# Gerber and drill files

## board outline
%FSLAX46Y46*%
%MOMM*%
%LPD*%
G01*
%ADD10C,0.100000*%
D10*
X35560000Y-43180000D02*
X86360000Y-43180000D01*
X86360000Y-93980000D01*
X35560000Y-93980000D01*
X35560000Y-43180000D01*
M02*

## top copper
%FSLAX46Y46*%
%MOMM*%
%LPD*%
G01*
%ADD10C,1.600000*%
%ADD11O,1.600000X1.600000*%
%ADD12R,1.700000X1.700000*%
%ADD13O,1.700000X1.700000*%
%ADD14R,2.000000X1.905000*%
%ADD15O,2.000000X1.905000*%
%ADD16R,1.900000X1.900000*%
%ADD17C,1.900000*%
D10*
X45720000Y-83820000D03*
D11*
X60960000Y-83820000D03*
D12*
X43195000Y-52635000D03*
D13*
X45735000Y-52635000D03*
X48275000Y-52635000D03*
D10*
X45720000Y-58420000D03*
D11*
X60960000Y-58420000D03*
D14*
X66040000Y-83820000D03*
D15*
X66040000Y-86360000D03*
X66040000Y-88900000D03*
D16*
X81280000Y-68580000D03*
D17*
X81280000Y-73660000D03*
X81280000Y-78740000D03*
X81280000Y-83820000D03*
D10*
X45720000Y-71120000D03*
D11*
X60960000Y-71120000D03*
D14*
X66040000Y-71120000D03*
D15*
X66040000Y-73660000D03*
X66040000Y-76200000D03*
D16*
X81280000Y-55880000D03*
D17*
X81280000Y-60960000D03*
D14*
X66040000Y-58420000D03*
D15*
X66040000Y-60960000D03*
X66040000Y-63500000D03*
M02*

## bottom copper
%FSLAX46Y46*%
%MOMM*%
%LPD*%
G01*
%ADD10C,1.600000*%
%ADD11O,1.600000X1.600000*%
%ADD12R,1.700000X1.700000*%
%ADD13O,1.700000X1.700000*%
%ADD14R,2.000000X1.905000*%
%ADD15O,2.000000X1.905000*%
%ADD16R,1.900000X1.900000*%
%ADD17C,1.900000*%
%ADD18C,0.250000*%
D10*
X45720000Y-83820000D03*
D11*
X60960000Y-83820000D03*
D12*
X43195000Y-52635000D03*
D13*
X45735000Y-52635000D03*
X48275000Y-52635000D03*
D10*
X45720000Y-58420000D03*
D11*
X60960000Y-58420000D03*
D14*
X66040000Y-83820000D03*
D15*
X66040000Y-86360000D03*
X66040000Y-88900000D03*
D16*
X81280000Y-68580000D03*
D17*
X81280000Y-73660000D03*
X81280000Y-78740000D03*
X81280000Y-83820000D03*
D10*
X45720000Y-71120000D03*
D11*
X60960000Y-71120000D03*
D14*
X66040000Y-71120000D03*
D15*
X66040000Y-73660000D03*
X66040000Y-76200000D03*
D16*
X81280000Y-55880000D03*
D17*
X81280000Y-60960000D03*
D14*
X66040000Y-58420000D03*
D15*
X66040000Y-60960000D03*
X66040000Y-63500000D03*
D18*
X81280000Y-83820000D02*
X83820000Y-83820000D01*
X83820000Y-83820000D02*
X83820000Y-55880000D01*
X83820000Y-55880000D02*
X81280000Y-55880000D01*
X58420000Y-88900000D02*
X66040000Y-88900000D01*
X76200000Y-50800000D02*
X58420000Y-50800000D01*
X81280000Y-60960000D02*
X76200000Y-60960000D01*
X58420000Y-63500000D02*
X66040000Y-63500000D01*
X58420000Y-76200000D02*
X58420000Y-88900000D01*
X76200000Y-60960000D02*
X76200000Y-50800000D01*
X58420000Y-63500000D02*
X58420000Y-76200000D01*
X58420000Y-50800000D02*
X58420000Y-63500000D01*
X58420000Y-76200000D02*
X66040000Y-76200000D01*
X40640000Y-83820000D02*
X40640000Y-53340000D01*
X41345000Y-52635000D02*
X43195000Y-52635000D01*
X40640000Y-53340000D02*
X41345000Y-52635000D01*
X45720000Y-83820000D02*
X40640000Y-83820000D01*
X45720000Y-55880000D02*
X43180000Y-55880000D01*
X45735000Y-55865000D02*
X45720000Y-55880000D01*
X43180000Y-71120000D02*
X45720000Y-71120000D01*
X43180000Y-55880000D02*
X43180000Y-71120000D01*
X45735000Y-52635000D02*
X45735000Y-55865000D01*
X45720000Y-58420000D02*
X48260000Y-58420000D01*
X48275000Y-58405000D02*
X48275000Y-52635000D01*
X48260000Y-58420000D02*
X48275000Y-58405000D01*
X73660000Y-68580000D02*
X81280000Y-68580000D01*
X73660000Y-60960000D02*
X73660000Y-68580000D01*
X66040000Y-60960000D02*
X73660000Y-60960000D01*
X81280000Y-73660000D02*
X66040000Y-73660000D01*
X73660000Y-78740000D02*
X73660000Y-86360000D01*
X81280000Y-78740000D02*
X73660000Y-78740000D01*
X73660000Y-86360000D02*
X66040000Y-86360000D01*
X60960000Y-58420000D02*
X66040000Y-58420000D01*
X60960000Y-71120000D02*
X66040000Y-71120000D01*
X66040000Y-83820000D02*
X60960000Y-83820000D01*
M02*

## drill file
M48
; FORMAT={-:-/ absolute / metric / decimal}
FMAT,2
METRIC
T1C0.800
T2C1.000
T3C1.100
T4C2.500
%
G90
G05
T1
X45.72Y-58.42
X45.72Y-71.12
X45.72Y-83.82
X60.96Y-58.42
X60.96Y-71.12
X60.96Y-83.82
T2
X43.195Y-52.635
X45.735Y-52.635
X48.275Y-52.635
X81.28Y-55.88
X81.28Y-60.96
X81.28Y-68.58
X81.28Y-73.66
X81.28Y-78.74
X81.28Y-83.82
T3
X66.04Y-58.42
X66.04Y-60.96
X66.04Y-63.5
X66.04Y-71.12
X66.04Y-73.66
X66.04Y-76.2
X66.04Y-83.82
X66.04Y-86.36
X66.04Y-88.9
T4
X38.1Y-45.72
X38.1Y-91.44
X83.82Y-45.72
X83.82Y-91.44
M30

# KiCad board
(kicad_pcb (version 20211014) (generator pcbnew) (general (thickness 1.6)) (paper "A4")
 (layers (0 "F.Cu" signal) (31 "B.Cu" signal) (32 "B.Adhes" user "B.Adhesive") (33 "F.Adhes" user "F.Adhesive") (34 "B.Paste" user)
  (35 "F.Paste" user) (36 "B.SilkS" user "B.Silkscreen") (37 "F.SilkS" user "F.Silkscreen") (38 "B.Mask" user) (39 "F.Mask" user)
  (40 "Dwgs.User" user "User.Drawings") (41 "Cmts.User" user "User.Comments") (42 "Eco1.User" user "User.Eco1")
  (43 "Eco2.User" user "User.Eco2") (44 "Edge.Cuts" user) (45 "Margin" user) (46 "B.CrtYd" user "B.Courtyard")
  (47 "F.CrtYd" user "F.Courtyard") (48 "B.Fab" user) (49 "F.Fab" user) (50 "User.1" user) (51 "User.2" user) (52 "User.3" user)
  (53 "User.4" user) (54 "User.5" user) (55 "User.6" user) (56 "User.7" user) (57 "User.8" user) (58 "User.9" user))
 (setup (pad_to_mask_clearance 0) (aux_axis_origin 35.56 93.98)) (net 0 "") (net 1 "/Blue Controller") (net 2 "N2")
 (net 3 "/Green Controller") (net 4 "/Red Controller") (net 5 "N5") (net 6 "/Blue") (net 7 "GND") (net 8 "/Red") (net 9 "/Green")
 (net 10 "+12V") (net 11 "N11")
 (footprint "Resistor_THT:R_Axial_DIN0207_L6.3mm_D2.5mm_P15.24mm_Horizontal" (layer "F.Cu") (at 45.72 83.82)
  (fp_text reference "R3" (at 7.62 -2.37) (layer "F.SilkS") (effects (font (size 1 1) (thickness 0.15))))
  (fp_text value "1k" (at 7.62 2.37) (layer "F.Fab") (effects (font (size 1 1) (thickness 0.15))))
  (pad "1" thru_hole circle (at 0 0) (size 1.6 1.6) (drill 0.8) (layers *.Cu *.Mask) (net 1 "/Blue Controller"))
  (pad "2" thru_hole oval (at 15.24 0) (size 1.6 1.6) (drill 0.8) (layers *.Cu *.Mask) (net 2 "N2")))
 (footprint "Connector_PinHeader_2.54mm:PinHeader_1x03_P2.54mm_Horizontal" (layer "F.Cu") (at 43.195 52.635 90)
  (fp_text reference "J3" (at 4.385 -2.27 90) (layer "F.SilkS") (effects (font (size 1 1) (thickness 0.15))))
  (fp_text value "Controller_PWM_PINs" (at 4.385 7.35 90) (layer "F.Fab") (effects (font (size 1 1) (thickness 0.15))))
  (pad "1" thru_hole rect (at 0 0 90) (size 1.7 1.7) (drill 1) (layers *.Cu *.Mask) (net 1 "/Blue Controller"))
  (pad "2" thru_hole oval (at 0 2.54 90) (size 1.7 1.7) (drill 1) (layers *.Cu *.Mask) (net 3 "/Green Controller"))
  (pad "3" thru_hole oval (at 0 5.08 90) (size 1.7 1.7) (drill 1) (layers *.Cu *.Mask) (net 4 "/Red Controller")))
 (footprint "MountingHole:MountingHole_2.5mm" (layer "F.Cu") (at 83.82 45.72)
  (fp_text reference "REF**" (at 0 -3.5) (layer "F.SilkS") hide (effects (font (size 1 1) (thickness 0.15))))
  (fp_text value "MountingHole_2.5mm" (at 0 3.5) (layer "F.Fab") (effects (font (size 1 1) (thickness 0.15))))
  (pad "" np_thru_hole circle (at 0 0) (size 2.5 2.5) (drill 2.5) (layers *.Cu *.Mask)))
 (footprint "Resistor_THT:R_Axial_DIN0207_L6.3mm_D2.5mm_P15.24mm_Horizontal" (layer "F.Cu") (at 45.72 58.42)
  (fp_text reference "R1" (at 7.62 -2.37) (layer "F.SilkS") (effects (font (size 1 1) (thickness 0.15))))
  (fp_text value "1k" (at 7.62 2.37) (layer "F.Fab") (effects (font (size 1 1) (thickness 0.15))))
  (pad "1" thru_hole circle (at 0 0) (size 1.6 1.6) (drill 0.8) (layers *.Cu *.Mask) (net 4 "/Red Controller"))
  (pad "2" thru_hole oval (at 15.24 0) (size 1.6 1.6) (drill 0.8) (layers *.Cu *.Mask) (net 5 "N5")))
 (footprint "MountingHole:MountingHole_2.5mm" (layer "F.Cu") (at 38.1 45.72)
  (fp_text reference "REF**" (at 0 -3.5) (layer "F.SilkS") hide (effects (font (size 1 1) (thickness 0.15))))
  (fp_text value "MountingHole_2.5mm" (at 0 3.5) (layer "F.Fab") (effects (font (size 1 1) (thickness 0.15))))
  (pad "" np_thru_hole circle (at 0 0) (size 2.5 2.5) (drill 2.5) (layers *.Mask)))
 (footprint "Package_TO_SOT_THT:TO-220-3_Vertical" (layer "F.Cu") (at 66.04 83.82 -90)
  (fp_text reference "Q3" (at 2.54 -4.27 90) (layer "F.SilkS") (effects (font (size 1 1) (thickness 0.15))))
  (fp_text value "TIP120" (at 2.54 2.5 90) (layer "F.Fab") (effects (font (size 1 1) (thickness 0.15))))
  (pad "1" thru_hole rect (at 0 0 270) (size 1.905 2) (drill 1.1) (layers *.Cu *.Mask) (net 2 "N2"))
  (pad "2" thru_hole oval (at 2.54 0 270) (size 1.905 2) (drill 1.1) (layers *.Cu *.Mask) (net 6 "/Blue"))
  (pad "3" thru_hole oval (at 5.08 0 270) (size 1.905 2) (drill 1.1) (layers *.Cu *.Mask) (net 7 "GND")))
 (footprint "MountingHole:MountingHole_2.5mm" (layer "F.Cu") (at 83.82 91.44)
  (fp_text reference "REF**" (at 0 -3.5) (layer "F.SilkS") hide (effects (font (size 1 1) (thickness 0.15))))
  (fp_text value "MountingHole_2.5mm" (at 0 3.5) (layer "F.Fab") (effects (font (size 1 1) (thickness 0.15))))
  (pad "" np_thru_hole circle (at 0 0) (size 2.5 2.5) (drill 2.5) (layers *.Cu *.Mask)))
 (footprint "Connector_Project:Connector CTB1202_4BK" (layer "F.Cu") (at 81.28 68.58 -90)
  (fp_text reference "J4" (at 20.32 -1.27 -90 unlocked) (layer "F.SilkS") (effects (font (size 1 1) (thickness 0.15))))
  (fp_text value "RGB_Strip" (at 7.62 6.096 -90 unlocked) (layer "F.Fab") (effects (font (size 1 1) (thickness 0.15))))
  (pad "1" thru_hole rect (at 0 0 270) (size 1.9 1.9) (drill 1) (layers *.Cu *.Mask) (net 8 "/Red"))
  (pad "2" thru_hole circle (at 5.08 0 270) (size 1.9 1.9) (drill 1) (layers *.Cu *.Mask) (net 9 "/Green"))
  (pad "3" thru_hole circle (at 10.16 0 270) (size 1.9 1.9) (drill 1) (layers *.Cu *.Mask) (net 6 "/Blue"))
  (pad "4" thru_hole circle (at 15.24 0 270) (size 1.9 1.9) (drill 1) (layers *.Cu *.Mask) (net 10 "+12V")))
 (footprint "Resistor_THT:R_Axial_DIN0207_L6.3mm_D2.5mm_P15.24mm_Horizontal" (layer "F.Cu") (at 45.72 71.12)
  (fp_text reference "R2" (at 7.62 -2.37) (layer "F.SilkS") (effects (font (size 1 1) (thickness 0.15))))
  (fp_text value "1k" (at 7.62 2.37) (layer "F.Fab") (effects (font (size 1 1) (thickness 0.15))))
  (pad "1" thru_hole circle (at 0 0) (size 1.6 1.6) (drill 0.8) (layers *.Cu *.Mask) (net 3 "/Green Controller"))
  (pad "2" thru_hole oval (at 15.24 0) (size 1.6 1.6) (drill 0.8) (layers *.Cu *.Mask) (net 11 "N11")))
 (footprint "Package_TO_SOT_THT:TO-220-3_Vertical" (layer "F.Cu") (at 66.04 71.12 -90)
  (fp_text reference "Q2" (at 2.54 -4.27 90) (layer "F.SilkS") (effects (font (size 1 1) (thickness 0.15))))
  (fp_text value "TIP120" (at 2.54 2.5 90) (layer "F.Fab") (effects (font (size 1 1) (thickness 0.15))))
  (pad "1" thru_hole rect (at 0 0 270) (size 1.905 2) (drill 1.1) (layers *.Cu *.Mask) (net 11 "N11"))
  (pad "2" thru_hole oval (at 2.54 0 270) (size 1.905 2) (drill 1.1) (layers *.Cu *.Mask) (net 9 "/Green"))
  (pad "3" thru_hole oval (at 5.08 0 270) (size 1.905 2) (drill 1.1) (layers *.Cu *.Mask) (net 7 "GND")))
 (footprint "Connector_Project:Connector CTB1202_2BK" (layer "F.Cu") (at 81.28 55.88 -90)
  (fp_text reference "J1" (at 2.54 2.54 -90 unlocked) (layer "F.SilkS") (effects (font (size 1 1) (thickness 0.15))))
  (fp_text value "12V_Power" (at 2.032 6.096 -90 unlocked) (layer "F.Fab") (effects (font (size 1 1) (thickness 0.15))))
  (pad "1" thru_hole rect (at 0 0 270) (size 1.9 1.9) (drill 1) (layers *.Cu *.Mask) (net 10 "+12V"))
  (pad "2" thru_hole circle (at 5.08 0 270) (size 1.9 1.9) (drill 1) (layers *.Cu *.Mask) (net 7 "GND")))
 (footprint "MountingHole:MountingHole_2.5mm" (layer "F.Cu") (at 38.1 91.44)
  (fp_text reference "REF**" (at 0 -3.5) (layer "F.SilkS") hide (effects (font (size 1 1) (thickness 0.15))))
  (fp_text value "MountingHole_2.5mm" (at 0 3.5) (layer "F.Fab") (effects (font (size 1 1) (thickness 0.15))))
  (pad "" np_thru_hole circle (at 0 0) (size 2.5 2.5) (drill 2.5) (layers *.Cu *.Mask)))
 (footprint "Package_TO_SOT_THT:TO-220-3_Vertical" (layer "F.Cu") (at 66.04 58.42 -90)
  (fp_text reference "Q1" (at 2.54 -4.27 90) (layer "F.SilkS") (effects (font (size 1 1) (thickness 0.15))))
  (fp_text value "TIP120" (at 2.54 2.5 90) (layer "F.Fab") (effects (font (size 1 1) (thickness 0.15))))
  (pad "1" thru_hole rect (at 0 0 270) (size 1.905 2) (drill 1.1) (layers *.Cu *.Mask) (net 5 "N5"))
  (pad "2" thru_hole oval (at 2.54 0 270) (size 1.905 2) (drill 1.1) (layers *.Cu *.Mask) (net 8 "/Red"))
  (pad "3" thru_hole oval (at 5.08 0 270) (size 1.905 2) (drill 1.1) (layers *.Cu *.Mask) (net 7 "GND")))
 (gr_rect (start 35.56 43.18) (end 86.36 93.98) (layer "Edge.Cuts") (width 0.1) (fill none))
 (segment (start 81.28 83.82) (end 83.82 83.82) (width 0.25) (layer "B.Cu") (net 10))
 (segment (start 83.82 83.82) (end 83.82 55.88) (width 0.25) (layer "B.Cu") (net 10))
 (segment (start 83.82 55.88) (end 81.28 55.88) (width 0.25) (layer "B.Cu") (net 10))
 (segment (start 58.42 88.9) (end 66.04 88.9) (width 0.25) (layer "B.Cu") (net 7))
 (segment (start 76.2 50.8) (end 58.42 50.8) (width 0.25) (layer "B.Cu") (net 7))
 (segment (start 81.28 60.96) (end 76.2 60.96) (width 0.25) (layer "B.Cu") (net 7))
 (segment (start 58.42 63.5) (end 66.04 63.5) (width 0.25) (layer "B.Cu") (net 7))
 (segment (start 58.42 76.2) (end 58.42 88.9) (width 0.25) (layer "B.Cu") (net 7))
 (segment (start 76.2 60.96) (end 76.2 50.8) (width 0.25) (layer "B.Cu") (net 7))
 (segment (start 58.42 63.5) (end 58.42 76.2) (width 0.25) (layer "B.Cu") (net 7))
 (segment (start 58.42 50.8) (end 58.42 63.5) (width 0.25) (layer "B.Cu") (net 7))
 (segment (start 58.42 76.2) (end 66.04 76.2) (width 0.25) (layer "B.Cu") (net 7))
 (segment (start 40.64 83.82) (end 40.64 53.34) (width 0.25) (layer "B.Cu") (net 1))
 (segment (start 41.345 52.635) (end 43.195 52.635) (width 0.25) (layer "B.Cu") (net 1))
 (segment (start 40.64 53.34) (end 41.345 52.635) (width 0.25) (layer "B.Cu") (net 1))
 (segment (start 45.72 83.82) (end 40.64 83.82) (width 0.25) (layer "B.Cu") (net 1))
 (segment (start 45.72 55.88) (end 43.18 55.88) (width 0.25) (layer "B.Cu") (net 3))
 (segment (start 45.735 55.865) (end 45.72 55.88) (width 0.25) (layer "B.Cu") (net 3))
 (segment (start 43.18 71.12) (end 45.72 71.12) (width 0.25) (layer "B.Cu") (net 3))
 (segment (start 43.18 55.88) (end 43.18 71.12) (width 0.25) (layer "B.Cu") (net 3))
 (segment (start 45.735 52.635) (end 45.735 55.865) (width 0.25) (layer "B.Cu") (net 3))
 (segment (start 45.72 58.42) (end 48.26 58.42) (width 0.25) (layer "B.Cu") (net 4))
 (segment (start 48.275 58.405) (end 48.275 52.635) (width 0.25) (layer "B.Cu") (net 4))
 (segment (start 48.26 58.42) (end 48.275 58.405) (width 0.25) (layer "B.Cu") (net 4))
 (segment (start 73.66 68.58) (end 81.28 68.58) (width 0.25) (layer "B.Cu") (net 8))
 (segment (start 73.66 60.96) (end 73.66 68.58) (width 0.25) (layer "B.Cu") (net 8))
 (segment (start 66.04 60.96) (end 73.66 60.96) (width 0.25) (layer "B.Cu") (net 8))
 (segment (start 81.28 73.66) (end 66.04 73.66) (width 0.25) (layer "B.Cu") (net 9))
 (segment (start 73.66 78.74) (end 73.66 86.36) (width 0.25) (layer "B.Cu") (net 6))
 (segment (start 81.28 78.74) (end 73.66 78.74) (width 0.25) (layer "B.Cu") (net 6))
 (segment (start 73.66 86.36) (end 66.04 86.36) (width 0.25) (layer "B.Cu") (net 6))
 (segment (start 60.96 58.42) (end 66.04 58.42) (width 0.25) (layer "B.Cu") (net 5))
 (segment (start 60.96 71.12) (end 66.04 71.12) (width 0.25) (layer "B.Cu") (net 11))
 (segment (start 66.04 83.82) (end 60.96 83.82) (width 0.25) (layer "B.Cu") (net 2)))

